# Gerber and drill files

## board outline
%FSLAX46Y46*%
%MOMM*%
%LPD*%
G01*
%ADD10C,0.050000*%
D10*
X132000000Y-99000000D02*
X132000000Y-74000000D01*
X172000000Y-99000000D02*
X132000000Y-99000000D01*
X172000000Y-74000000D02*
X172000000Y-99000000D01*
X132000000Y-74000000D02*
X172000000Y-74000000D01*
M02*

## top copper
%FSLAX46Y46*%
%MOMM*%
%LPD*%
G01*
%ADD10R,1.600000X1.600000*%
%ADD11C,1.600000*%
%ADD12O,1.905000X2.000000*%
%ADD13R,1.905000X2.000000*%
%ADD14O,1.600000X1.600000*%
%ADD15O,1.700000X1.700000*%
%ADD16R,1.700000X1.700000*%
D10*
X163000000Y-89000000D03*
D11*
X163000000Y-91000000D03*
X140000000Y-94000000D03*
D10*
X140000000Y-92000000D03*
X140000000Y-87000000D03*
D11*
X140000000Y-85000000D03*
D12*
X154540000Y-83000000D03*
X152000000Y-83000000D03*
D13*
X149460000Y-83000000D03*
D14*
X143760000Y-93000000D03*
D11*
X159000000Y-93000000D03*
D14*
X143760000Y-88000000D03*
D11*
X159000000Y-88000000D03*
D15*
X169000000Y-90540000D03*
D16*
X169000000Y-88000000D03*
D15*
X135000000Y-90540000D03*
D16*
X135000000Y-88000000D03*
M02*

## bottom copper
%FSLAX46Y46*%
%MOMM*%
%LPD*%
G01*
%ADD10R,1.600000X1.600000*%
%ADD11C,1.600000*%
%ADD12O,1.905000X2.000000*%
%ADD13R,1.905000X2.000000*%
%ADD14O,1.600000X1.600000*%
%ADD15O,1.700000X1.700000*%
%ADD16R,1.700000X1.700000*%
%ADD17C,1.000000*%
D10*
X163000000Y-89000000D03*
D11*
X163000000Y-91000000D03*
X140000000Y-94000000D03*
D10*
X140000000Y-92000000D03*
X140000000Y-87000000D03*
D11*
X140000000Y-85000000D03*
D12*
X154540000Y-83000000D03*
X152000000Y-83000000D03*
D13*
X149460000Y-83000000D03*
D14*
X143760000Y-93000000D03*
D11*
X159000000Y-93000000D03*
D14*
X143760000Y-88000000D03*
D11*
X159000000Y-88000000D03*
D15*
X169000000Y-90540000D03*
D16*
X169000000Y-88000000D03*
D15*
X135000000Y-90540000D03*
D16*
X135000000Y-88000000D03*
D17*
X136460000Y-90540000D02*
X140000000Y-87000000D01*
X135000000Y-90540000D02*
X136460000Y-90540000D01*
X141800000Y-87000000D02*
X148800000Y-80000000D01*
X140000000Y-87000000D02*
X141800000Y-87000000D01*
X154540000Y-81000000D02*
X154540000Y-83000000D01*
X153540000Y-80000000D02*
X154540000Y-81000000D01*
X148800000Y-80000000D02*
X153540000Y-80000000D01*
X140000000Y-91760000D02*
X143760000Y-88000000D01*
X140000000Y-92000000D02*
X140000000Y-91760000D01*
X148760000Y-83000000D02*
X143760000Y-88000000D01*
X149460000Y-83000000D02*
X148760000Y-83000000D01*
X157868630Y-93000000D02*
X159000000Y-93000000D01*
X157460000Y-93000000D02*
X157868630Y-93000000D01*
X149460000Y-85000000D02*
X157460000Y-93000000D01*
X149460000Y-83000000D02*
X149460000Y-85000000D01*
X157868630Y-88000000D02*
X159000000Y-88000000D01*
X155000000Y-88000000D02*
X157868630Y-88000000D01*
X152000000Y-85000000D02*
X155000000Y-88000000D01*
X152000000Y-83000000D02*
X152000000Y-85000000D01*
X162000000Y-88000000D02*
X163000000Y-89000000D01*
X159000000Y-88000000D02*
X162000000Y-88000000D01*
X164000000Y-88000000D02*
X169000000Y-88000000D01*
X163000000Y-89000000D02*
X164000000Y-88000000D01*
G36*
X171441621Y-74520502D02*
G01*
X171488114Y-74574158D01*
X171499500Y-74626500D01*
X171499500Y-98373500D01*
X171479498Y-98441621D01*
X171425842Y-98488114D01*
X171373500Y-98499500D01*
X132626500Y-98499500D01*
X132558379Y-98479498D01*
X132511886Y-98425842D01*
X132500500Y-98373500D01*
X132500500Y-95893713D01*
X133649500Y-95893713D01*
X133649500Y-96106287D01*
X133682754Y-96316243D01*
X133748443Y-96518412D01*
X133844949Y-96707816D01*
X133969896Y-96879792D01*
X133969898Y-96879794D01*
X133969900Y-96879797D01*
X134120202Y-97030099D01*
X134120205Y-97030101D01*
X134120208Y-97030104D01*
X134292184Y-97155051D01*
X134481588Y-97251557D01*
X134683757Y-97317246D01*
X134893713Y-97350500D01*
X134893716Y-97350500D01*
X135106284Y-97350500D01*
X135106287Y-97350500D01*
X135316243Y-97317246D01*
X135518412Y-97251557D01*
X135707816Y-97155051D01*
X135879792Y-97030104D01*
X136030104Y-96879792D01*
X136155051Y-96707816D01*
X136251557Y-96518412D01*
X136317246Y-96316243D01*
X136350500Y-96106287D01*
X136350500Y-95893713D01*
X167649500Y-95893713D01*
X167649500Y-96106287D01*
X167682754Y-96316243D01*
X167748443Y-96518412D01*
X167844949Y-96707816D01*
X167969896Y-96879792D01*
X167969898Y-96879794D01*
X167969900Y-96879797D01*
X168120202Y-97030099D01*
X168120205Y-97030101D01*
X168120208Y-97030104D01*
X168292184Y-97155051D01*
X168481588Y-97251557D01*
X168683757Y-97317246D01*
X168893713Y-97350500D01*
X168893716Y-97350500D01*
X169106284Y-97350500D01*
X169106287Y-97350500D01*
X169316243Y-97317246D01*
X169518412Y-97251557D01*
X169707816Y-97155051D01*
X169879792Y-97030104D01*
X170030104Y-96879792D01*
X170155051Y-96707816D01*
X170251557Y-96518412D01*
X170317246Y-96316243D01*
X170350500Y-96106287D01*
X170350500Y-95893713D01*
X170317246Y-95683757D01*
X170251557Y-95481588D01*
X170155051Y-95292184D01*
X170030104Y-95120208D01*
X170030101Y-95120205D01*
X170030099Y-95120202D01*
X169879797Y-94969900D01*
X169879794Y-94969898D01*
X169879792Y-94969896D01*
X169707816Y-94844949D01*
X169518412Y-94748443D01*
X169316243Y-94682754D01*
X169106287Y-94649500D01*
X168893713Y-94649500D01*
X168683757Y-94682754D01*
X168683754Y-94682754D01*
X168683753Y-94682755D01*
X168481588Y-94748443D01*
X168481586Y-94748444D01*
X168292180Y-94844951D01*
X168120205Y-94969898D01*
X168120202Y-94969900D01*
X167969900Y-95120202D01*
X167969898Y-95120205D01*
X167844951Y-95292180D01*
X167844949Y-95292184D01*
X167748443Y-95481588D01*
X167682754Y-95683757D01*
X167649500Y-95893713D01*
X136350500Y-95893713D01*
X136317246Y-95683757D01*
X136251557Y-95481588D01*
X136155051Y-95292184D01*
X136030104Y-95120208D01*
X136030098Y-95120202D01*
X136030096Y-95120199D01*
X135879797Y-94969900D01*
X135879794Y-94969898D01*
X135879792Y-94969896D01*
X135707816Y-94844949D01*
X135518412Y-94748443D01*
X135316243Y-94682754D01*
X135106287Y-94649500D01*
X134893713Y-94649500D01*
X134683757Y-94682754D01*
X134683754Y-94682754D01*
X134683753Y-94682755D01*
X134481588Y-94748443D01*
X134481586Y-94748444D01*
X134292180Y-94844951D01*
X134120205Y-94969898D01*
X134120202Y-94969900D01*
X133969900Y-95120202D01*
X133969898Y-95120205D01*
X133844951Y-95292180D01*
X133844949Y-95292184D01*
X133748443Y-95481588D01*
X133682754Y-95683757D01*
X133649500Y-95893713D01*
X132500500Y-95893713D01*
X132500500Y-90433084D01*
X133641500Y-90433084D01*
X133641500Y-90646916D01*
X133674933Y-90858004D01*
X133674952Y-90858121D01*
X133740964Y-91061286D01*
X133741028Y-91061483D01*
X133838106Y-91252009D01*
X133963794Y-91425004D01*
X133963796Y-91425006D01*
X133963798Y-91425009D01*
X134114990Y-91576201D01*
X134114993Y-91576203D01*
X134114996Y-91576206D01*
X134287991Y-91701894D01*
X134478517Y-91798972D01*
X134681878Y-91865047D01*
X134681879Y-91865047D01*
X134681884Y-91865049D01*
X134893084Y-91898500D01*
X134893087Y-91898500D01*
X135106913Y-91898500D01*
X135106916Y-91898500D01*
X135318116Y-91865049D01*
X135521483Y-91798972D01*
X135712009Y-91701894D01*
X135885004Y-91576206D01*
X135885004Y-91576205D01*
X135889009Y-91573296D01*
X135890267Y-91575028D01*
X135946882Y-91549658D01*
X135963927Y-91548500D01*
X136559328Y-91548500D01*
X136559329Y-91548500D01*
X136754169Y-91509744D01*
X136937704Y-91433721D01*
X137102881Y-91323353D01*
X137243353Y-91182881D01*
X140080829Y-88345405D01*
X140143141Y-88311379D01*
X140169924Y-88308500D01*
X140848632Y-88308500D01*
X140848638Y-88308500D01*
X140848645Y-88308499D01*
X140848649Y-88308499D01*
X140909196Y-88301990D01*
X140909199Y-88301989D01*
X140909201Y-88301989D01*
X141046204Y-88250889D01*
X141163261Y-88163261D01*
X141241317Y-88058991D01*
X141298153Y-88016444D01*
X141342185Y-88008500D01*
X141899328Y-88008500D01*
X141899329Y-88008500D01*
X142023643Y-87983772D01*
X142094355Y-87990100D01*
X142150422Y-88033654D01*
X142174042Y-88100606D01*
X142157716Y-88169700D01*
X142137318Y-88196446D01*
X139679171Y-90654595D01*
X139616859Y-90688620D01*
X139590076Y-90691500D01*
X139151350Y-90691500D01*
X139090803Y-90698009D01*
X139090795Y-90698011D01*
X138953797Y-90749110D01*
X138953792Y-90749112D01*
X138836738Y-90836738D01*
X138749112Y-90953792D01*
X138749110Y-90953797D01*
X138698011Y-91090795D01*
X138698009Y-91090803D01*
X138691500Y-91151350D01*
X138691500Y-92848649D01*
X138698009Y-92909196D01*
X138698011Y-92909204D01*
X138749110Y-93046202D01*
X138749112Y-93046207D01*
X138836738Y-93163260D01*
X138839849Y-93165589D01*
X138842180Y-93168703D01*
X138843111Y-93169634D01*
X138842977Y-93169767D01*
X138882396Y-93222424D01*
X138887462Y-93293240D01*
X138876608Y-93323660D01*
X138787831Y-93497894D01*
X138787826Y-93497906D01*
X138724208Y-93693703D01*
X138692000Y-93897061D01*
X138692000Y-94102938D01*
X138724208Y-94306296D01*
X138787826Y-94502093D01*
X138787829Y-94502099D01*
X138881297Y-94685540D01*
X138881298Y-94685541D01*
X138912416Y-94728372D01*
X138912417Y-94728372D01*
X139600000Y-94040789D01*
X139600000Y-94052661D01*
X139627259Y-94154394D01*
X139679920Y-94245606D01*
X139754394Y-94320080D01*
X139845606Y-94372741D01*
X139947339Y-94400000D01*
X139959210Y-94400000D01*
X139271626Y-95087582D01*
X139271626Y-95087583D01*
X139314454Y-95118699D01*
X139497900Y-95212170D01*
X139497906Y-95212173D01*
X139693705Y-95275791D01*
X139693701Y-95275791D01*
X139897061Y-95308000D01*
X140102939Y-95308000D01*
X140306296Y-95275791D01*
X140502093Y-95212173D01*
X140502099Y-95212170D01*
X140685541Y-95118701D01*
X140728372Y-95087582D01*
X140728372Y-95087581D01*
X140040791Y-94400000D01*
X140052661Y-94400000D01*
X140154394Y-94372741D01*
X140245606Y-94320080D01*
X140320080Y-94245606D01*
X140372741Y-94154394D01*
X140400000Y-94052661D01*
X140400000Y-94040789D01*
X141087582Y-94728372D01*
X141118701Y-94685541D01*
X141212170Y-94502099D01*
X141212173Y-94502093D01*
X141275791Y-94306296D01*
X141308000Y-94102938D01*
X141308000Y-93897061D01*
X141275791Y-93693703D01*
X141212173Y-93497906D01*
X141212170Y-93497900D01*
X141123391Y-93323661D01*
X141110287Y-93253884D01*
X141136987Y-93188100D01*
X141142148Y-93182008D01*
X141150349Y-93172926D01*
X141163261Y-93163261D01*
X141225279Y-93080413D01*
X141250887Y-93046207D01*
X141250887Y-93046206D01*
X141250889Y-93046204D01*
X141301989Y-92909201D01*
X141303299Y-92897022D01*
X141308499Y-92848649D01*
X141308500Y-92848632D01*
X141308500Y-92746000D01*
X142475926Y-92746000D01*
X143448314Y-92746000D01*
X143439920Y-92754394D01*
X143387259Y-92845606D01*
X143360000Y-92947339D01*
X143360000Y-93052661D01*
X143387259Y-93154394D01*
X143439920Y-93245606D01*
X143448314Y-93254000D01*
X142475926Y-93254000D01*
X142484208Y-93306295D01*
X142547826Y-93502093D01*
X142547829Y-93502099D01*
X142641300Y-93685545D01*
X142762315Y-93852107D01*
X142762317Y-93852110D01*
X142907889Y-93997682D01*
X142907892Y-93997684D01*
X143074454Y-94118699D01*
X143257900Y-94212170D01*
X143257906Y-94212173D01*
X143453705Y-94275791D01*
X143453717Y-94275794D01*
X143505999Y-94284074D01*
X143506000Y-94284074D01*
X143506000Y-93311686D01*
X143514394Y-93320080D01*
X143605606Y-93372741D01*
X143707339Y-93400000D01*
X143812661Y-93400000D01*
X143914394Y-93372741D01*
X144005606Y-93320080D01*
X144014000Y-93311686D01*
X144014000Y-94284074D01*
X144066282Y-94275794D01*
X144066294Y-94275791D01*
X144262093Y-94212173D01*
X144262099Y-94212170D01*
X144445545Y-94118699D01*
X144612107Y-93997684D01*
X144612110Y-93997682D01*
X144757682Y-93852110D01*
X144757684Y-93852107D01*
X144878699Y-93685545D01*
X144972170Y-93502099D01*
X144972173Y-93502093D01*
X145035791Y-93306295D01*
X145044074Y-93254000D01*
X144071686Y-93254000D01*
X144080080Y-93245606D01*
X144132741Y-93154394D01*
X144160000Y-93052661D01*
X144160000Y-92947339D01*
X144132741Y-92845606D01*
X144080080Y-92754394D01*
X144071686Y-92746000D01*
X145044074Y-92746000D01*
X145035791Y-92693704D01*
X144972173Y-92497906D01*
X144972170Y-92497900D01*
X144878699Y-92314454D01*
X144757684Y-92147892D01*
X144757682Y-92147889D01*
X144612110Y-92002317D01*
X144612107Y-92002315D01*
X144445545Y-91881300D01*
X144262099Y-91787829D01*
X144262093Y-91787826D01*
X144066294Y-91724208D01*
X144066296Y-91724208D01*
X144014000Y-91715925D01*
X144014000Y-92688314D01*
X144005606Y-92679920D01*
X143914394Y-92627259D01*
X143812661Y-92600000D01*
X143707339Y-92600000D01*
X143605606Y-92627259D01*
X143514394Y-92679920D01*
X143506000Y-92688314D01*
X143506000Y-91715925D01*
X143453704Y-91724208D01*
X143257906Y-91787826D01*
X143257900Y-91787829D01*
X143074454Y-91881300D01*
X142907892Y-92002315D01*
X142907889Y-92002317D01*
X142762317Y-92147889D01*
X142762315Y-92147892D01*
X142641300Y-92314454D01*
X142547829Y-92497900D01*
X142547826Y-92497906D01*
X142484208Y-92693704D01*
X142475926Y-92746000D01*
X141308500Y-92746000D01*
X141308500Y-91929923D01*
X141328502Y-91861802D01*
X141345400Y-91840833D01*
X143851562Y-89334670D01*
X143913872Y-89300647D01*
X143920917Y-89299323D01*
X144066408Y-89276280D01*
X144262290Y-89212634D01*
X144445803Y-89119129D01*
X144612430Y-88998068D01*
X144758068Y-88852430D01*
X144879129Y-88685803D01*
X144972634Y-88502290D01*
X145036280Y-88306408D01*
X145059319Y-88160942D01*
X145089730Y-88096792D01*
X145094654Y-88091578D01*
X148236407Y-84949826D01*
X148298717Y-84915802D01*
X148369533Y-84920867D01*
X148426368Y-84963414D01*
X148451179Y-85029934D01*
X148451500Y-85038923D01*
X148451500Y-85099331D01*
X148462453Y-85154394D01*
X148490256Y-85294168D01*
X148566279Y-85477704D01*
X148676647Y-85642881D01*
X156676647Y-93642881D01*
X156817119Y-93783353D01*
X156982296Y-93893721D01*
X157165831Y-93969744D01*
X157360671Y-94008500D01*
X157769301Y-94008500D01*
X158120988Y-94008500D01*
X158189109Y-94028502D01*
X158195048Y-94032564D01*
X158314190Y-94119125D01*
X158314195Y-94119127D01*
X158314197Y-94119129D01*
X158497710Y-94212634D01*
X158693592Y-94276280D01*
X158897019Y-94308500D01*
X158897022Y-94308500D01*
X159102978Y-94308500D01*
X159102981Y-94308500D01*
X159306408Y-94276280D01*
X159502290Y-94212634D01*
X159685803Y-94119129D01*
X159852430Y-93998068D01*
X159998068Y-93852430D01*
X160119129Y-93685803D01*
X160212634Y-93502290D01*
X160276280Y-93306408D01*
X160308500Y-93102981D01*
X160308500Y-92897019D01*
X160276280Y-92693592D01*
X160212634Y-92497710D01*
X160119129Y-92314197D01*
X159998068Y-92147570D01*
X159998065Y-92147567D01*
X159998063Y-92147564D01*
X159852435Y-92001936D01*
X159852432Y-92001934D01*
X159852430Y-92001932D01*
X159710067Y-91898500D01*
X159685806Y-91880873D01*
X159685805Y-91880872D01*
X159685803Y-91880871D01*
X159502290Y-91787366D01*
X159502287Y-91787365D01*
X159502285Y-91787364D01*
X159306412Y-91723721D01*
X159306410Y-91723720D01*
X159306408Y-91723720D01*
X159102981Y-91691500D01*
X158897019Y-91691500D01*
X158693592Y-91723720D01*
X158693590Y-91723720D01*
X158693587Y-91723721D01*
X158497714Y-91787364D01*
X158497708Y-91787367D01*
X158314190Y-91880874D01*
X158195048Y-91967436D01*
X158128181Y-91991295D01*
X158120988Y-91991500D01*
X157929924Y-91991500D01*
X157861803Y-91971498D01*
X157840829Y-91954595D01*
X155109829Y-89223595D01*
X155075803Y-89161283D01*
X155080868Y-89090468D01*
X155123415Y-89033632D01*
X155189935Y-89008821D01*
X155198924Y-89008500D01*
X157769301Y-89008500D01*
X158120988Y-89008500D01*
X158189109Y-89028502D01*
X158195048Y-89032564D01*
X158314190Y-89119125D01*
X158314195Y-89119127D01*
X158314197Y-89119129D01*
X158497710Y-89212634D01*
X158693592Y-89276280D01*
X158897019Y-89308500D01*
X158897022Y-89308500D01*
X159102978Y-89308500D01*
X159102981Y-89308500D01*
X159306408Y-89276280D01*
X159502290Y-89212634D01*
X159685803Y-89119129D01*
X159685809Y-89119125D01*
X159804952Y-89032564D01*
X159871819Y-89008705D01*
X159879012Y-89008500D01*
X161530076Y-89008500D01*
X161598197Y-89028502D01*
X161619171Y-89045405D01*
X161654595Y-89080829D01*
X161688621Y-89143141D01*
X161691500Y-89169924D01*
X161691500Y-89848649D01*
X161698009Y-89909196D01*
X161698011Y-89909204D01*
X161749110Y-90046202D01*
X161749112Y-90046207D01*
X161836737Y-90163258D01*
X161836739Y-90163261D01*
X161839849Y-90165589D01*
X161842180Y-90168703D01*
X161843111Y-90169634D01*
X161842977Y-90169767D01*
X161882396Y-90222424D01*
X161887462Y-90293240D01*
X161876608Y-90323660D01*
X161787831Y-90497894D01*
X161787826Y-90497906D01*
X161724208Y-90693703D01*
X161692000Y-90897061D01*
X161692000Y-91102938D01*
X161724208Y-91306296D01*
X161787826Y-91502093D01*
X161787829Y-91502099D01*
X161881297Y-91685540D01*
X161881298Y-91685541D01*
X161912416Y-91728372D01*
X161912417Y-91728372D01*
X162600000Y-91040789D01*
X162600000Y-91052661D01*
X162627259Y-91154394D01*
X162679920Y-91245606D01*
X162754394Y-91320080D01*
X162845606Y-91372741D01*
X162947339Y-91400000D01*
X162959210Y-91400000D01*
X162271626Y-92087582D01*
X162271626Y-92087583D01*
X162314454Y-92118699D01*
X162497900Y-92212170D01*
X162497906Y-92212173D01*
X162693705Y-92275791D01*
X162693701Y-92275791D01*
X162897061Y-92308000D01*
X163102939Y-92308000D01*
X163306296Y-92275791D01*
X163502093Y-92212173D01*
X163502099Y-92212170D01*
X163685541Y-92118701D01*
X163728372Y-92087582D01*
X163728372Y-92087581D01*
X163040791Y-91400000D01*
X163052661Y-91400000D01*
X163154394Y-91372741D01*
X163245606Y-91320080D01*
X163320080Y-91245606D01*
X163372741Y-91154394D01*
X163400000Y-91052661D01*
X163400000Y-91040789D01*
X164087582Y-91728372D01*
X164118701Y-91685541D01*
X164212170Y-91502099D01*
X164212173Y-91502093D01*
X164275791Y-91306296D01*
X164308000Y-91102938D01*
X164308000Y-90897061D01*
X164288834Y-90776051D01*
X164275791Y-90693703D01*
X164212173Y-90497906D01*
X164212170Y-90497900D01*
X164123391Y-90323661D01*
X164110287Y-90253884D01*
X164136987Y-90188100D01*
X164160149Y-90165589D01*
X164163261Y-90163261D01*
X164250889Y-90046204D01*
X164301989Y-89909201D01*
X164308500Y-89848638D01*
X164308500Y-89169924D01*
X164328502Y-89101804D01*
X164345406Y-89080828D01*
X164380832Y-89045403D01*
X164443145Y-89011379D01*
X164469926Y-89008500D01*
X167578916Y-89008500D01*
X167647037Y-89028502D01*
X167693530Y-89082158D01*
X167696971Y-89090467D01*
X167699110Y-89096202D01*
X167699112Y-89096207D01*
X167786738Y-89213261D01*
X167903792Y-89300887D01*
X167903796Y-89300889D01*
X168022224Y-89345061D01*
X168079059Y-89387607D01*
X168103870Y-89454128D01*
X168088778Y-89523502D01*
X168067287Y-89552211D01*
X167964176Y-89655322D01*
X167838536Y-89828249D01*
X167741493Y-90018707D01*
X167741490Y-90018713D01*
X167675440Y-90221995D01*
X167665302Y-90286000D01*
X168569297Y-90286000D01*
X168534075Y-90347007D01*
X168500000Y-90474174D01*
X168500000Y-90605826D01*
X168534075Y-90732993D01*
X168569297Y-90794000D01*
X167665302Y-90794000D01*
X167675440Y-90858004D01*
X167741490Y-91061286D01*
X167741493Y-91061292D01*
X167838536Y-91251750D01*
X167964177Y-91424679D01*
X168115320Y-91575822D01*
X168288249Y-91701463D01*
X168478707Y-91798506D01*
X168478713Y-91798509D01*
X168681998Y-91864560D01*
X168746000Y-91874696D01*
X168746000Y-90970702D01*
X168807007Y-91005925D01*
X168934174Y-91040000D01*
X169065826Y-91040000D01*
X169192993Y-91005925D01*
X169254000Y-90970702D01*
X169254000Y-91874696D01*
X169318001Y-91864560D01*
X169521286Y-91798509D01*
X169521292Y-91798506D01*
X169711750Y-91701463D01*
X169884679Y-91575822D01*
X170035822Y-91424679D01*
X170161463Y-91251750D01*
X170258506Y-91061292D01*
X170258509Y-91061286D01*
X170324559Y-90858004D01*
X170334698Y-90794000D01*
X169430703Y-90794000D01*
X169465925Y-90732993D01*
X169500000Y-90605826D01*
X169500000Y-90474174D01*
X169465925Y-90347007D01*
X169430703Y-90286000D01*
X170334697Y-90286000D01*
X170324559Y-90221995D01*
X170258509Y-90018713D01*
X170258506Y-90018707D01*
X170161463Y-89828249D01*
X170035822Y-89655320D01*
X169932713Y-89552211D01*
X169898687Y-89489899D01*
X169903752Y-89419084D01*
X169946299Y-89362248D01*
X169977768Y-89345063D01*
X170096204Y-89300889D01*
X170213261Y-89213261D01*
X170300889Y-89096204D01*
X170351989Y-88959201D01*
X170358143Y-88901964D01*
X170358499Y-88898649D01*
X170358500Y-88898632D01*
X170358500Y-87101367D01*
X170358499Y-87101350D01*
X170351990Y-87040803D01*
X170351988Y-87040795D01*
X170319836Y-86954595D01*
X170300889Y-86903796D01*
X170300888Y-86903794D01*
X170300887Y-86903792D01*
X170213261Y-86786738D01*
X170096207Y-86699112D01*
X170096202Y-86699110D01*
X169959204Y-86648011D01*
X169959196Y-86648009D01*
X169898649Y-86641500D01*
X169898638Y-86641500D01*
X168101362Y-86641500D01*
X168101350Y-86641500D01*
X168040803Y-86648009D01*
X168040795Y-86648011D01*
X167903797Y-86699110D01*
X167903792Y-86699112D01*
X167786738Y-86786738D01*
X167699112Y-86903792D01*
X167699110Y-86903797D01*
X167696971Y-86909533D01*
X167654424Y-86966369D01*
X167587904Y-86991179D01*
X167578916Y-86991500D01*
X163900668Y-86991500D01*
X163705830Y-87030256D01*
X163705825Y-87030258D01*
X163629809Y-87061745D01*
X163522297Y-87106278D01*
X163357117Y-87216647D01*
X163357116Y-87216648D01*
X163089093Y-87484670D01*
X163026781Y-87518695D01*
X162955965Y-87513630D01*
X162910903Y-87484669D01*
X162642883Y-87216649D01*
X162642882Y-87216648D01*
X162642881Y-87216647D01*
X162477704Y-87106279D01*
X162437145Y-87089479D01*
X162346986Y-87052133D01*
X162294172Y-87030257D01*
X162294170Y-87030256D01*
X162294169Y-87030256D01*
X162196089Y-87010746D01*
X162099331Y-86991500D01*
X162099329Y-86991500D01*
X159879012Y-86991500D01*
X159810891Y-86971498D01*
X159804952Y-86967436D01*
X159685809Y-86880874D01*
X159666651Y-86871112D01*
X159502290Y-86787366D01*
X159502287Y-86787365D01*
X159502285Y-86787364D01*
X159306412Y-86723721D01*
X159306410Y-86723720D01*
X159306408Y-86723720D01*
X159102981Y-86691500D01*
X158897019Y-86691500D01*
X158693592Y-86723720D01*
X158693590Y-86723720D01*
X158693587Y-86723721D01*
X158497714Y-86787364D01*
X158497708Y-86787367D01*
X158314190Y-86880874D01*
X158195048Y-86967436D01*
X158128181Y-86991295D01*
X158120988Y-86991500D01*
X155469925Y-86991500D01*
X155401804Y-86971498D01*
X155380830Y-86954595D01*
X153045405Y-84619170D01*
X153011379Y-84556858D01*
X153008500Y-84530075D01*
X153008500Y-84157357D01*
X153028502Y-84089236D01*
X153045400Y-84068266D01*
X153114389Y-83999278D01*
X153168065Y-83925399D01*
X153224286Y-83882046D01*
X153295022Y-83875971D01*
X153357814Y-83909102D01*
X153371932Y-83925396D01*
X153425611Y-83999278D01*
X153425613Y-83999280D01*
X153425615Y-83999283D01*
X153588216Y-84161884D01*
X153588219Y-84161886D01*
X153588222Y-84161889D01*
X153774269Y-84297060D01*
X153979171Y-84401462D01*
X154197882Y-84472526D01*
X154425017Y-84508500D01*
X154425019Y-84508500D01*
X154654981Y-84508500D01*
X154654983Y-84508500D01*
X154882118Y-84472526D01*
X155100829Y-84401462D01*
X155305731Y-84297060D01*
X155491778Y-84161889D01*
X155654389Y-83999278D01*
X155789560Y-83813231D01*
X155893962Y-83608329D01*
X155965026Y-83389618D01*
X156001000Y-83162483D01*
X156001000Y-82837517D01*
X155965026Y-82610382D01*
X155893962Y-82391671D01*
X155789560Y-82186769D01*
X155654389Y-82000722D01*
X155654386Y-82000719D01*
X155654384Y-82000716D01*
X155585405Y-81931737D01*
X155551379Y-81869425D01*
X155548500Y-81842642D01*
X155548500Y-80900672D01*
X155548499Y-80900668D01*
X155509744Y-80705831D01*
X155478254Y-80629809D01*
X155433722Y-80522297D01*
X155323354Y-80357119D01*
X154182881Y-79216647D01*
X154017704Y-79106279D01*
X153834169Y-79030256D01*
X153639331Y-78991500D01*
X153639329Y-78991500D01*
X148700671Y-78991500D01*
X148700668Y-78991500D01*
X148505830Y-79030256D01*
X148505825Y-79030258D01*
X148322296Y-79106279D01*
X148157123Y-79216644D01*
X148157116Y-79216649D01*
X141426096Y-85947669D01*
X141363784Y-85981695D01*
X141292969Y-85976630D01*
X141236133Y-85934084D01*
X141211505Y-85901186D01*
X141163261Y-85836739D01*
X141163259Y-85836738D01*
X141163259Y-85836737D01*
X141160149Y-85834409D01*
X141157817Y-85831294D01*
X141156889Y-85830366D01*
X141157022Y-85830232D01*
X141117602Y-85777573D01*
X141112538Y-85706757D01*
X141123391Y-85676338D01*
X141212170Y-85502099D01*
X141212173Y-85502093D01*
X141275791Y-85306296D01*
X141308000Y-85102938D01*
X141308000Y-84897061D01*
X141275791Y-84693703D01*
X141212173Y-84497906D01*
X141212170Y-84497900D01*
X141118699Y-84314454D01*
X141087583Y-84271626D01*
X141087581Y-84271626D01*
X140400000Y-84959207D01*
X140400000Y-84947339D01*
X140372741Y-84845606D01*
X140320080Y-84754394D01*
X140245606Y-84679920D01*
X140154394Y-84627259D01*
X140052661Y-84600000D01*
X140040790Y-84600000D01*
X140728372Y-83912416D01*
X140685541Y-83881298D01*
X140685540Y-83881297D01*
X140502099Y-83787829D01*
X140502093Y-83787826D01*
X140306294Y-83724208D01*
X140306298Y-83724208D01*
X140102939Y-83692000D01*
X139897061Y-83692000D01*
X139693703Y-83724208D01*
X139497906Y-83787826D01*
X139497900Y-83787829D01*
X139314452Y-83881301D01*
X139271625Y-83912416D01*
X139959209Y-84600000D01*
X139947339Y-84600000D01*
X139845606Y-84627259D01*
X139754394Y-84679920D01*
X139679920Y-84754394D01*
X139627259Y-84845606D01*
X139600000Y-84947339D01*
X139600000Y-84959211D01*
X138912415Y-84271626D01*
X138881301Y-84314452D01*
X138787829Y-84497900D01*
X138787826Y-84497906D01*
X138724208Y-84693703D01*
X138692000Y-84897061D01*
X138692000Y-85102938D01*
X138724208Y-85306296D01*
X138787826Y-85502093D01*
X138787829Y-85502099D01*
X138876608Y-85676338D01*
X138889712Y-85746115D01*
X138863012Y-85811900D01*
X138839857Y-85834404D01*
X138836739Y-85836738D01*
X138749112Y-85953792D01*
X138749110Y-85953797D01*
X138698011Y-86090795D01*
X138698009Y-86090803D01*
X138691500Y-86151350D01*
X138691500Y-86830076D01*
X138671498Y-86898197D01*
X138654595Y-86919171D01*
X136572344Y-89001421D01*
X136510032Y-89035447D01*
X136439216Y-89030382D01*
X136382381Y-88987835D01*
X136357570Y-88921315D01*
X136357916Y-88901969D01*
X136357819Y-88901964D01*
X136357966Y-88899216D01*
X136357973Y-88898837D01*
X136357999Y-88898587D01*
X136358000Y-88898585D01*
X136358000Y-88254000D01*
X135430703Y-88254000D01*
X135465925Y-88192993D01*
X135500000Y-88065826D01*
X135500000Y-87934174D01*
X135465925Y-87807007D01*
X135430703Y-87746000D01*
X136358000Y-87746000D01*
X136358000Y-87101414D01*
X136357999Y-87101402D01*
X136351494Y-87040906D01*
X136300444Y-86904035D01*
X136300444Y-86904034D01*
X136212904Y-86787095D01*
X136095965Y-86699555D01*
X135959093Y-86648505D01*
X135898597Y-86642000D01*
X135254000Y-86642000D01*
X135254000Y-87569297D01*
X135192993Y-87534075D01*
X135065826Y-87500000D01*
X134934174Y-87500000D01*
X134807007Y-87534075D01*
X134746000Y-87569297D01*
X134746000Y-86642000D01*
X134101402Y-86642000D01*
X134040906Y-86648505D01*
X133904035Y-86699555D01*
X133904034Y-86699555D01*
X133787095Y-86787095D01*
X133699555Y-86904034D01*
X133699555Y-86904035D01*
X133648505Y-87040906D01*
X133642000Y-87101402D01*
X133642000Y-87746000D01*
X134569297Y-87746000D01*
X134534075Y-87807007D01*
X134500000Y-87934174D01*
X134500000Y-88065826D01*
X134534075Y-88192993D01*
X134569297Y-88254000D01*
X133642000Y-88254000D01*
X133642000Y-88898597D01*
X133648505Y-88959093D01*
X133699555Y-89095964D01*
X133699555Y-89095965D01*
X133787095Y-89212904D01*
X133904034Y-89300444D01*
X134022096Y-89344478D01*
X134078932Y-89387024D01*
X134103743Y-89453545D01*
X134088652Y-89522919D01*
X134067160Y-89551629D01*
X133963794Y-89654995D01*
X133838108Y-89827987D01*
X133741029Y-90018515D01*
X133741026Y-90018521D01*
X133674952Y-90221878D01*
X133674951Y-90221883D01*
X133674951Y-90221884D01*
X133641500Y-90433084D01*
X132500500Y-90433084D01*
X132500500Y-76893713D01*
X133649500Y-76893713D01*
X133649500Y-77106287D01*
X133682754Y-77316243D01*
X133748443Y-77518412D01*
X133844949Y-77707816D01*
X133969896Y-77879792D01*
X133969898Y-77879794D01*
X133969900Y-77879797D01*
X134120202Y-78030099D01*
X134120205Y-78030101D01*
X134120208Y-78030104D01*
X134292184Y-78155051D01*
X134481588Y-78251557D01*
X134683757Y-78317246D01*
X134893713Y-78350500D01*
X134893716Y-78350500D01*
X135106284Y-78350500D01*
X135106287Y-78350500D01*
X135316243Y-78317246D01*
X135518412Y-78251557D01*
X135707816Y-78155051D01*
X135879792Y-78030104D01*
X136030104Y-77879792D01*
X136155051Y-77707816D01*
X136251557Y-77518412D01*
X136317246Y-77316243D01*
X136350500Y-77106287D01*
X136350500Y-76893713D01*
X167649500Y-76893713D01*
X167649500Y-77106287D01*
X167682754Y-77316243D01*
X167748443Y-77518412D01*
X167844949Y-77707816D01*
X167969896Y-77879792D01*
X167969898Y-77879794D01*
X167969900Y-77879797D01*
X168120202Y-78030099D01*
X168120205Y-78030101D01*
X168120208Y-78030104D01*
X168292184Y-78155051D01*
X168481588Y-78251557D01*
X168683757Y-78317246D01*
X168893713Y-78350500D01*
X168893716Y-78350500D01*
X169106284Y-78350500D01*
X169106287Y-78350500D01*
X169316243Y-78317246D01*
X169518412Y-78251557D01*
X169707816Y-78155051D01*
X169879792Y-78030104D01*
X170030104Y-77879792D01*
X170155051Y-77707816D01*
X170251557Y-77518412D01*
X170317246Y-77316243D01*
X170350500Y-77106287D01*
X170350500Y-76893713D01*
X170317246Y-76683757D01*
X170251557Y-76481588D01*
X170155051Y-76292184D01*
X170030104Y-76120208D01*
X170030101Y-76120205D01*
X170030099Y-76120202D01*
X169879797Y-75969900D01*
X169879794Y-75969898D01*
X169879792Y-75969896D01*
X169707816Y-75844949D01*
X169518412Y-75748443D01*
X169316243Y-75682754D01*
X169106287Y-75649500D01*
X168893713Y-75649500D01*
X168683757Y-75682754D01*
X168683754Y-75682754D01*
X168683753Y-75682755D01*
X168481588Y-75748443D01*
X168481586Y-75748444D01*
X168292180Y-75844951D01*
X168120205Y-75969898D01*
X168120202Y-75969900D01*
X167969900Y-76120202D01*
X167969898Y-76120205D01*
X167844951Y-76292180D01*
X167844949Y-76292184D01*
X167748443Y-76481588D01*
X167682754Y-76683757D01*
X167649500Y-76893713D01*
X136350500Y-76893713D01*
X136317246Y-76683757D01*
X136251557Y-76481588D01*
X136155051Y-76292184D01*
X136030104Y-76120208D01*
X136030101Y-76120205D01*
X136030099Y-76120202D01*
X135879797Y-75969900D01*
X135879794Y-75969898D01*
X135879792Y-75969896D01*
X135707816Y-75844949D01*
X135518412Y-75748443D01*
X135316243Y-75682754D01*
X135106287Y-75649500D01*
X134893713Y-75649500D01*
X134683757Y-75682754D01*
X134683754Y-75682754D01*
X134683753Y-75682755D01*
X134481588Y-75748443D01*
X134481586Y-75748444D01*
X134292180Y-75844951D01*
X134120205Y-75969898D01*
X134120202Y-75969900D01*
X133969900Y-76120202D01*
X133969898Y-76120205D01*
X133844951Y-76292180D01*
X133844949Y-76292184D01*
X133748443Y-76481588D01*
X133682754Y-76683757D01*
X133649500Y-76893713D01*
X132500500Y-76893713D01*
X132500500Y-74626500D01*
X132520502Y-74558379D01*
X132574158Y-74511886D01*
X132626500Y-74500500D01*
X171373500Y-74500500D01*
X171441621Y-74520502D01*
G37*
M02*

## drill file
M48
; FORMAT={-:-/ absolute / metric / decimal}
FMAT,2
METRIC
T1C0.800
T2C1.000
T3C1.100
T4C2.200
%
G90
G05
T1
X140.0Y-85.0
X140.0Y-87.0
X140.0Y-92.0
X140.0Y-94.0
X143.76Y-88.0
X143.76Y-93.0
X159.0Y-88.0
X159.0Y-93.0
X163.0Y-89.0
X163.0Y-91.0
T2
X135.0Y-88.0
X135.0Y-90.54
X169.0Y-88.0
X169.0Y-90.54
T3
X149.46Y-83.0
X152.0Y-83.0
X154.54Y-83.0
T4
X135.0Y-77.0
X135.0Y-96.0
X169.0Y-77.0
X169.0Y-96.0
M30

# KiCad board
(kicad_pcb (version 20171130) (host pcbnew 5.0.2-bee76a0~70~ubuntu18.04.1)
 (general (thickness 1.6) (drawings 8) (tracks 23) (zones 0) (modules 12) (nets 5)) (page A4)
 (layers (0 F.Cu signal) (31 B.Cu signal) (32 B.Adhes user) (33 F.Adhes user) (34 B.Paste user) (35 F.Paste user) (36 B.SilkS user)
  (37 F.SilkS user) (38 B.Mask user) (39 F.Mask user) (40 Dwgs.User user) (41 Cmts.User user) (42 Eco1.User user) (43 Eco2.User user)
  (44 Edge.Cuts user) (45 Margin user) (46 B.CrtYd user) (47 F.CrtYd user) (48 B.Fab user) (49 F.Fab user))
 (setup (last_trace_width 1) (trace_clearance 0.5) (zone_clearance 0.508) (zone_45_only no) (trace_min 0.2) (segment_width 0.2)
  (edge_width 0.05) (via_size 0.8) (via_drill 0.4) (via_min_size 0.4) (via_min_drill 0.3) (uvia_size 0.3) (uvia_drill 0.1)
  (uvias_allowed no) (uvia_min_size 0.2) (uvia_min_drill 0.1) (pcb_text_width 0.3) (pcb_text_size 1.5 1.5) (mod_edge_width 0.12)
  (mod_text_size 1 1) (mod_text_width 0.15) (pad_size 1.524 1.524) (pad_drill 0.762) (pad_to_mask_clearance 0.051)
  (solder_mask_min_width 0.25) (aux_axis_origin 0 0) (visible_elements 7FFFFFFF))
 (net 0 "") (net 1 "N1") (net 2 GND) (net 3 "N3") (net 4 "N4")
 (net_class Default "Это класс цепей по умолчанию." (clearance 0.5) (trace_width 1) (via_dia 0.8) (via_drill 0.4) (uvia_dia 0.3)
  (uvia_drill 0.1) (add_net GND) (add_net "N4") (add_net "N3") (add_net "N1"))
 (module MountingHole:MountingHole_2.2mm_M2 (layer F.Cu) (at 169 77)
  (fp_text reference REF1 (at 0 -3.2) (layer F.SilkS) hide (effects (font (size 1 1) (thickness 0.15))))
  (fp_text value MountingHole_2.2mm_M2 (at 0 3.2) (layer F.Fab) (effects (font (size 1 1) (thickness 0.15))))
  (pad 1 np_thru_hole circle (at 0 0) (size 2.2 2.2) (drill 2.2) (layers *.Cu *.Mask)))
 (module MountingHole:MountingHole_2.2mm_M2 (layer F.Cu) (at 169 96)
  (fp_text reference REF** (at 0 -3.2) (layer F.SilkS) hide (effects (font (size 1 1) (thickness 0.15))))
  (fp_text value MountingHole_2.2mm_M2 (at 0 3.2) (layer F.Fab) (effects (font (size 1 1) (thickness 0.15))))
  (pad 1 np_thru_hole circle (at 0 0) (size 2.2 2.2) (drill 2.2) (layers *.Cu *.Mask)))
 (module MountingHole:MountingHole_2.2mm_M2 (layer F.Cu) (at 135 77)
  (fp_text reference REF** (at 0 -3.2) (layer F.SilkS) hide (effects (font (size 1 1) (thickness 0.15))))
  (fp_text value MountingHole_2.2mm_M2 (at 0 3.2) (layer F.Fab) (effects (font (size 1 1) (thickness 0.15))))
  (pad 1 np_thru_hole circle (at 0 0) (size 2.2 2.2) (drill 2.2) (layers *.Cu *.Mask)))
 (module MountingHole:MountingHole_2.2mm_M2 (layer F.Cu) (at 135 96)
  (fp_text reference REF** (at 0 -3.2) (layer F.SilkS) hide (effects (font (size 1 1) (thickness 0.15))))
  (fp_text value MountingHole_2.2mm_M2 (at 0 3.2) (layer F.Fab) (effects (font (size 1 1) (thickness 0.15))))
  (pad 1 np_thru_hole circle (at 0 0) (size 2.2 2.2) (drill 2.2) (layers *.Cu *.Mask)))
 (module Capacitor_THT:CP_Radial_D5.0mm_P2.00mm (layer F.Cu) (at 163 89 270)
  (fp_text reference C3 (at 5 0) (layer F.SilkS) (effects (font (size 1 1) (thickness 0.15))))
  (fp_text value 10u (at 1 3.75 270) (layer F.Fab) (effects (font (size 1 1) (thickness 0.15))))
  (pad 1 thru_hole rect (at 0 0 270) (size 1.6 1.6) (drill 0.8) (layers *.Cu *.Mask) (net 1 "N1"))
  (pad 2 thru_hole circle (at 2 0 270) (size 1.6 1.6) (drill 0.8) (layers *.Cu *.Mask) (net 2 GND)))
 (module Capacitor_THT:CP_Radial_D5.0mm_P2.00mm (layer F.Cu) (at 140 92 270)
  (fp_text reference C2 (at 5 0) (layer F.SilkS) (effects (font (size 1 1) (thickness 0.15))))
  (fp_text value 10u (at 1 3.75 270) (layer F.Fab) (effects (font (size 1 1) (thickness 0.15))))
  (pad 2 thru_hole circle (at 2 0 270) (size 1.6 1.6) (drill 0.8) (layers *.Cu *.Mask) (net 2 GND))
  (pad 1 thru_hole rect (at 0 0 270) (size 1.6 1.6) (drill 0.8) (layers *.Cu *.Mask) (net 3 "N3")))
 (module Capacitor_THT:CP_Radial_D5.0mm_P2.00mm (layer F.Cu) (at 140 87 90)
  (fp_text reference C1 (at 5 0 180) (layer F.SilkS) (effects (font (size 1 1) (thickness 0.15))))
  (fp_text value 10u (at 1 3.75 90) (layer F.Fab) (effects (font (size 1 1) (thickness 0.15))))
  (pad 1 thru_hole rect (at 0 0 90) (size 1.6 1.6) (drill 0.8) (layers *.Cu *.Mask) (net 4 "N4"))
  (pad 2 thru_hole circle (at 2 0 90) (size 1.6 1.6) (drill 0.8) (layers *.Cu *.Mask) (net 2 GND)))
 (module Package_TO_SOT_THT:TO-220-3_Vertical (layer F.Cu) (at 149.46 83)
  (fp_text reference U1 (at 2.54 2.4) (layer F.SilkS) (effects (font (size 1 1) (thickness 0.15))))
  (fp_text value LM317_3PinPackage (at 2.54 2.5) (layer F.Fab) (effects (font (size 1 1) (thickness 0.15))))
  (pad 3 thru_hole oval (at 5.08 0) (size 1.905 2) (drill 1.1) (layers *.Cu *.Mask) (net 4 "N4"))
  (pad 2 thru_hole oval (at 2.54 0) (size 1.905 2) (drill 1.1) (layers *.Cu *.Mask) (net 1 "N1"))
  (pad 1 thru_hole rect (at 0 0) (size 1.905 2) (drill 1.1) (layers *.Cu *.Mask) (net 3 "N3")))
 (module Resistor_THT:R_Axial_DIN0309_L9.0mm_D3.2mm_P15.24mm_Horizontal (layer F.Cu) (at 159 93 180)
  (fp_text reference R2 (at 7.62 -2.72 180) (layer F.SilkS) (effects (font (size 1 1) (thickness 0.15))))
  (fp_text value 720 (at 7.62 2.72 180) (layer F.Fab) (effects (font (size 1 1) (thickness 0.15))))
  (pad 2 thru_hole oval (at 15.24 0 180) (size 1.6 1.6) (drill 0.8) (layers *.Cu *.Mask) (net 2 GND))
  (pad 1 thru_hole circle (at 0 0 180) (size 1.6 1.6) (drill 0.8) (layers *.Cu *.Mask) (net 3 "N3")))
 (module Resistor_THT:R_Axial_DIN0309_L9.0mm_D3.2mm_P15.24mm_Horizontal (layer F.Cu) (at 159 88 180)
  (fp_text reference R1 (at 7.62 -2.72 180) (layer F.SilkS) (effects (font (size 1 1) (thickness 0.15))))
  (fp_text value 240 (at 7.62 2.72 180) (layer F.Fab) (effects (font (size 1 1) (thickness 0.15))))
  (pad 2 thru_hole oval (at 15.24 0 180) (size 1.6 1.6) (drill 0.8) (layers *.Cu *.Mask) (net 3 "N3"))
  (pad 1 thru_hole circle (at 0 0 180) (size 1.6 1.6) (drill 0.8) (layers *.Cu *.Mask) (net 1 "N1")))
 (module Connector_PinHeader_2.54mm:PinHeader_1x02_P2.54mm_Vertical (layer F.Cu) (at 169 88)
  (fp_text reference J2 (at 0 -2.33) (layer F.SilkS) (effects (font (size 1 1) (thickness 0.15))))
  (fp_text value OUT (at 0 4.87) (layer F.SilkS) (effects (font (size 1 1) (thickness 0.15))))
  (pad 2 thru_hole oval (at 0 2.54) (size 1.7 1.7) (drill 1) (layers *.Cu *.Mask) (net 2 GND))
  (pad 1 thru_hole rect (at 0 0) (size 1.7 1.7) (drill 1) (layers *.Cu *.Mask) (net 1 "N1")))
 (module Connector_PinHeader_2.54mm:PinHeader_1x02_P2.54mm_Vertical (layer F.Cu) (at 135 88)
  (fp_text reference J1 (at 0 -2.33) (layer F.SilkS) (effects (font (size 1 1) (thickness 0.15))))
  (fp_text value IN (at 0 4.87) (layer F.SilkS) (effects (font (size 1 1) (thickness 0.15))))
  (pad 2 thru_hole oval (at 0 2.54) (size 1.7 1.7) (drill 1) (layers *.Cu *.Mask) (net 4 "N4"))
  (pad 1 thru_hole rect (at 0 0) (size 1.7 1.7) (drill 1) (layers *.Cu *.Mask) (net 2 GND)))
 (gr_line (start 132 99) (end 132 74) (layer Edge.Cuts) (width 0.05))
 (gr_line (start 172 99) (end 132 99) (layer Edge.Cuts) (width 0.05))
 (gr_line (start 172 74) (end 172 99) (layer Edge.Cuts) (width 0.05))
 (gr_line (start 132 74) (end 172 74) (layer Edge.Cuts) (width 0.05))
 (segment (start 136.46 90.54) (end 140 87) (width 1) (layer B.Cu) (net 4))
 (segment (start 135 90.54) (end 136.46 90.54) (width 1) (layer B.Cu) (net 4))
 (segment (start 141.8 87) (end 148.8 80) (width 1) (layer B.Cu) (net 4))
 (segment (start 140 87) (end 141.8 87) (width 1) (layer B.Cu) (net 4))
 (segment (start 154.54 81) (end 154.54 83) (width 1) (layer B.Cu) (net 4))
 (segment (start 153.54 80) (end 154.54 81) (width 1) (layer B.Cu) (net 4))
 (segment (start 148.8 80) (end 153.54 80) (width 1) (layer B.Cu) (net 4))
 (segment (start 140 91.76) (end 143.76 88) (width 1) (layer B.Cu) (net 3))
 (segment (start 140 92) (end 140 91.76) (width 1) (layer B.Cu) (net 3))
 (segment (start 148.76 83) (end 143.76 88) (width 1) (layer B.Cu) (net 3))
 (segment (start 149.46 83) (end 148.76 83) (width 1) (layer B.Cu) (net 3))
 (segment (start 157.86863 93) (end 159 93) (width 1) (layer B.Cu) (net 3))
 (segment (start 157.46 93) (end 157.86863 93) (width 1) (layer B.Cu) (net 3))
 (segment (start 149.46 85) (end 157.46 93) (width 1) (layer B.Cu) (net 3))
 (segment (start 149.46 83) (end 149.46 85) (width 1) (layer B.Cu) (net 3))
 (segment (start 157.86863 88) (end 159 88) (width 1) (layer B.Cu) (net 1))
 (segment (start 155 88) (end 157.86863 88) (width 1) (layer B.Cu) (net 1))
 (segment (start 152 85) (end 155 88) (width 1) (layer B.Cu) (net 1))
 (segment (start 152 83) (end 152 85) (width 1) (layer B.Cu) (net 1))
 (segment (start 162 88) (end 163 89) (width 1) (layer B.Cu) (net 1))
 (segment (start 159 88) (end 162 88) (width 1) (layer B.Cu) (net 1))
 (segment (start 164 88) (end 169 88) (width 1) (layer B.Cu) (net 1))
 (segment (start 163 89) (end 164 88) (width 1) (layer B.Cu) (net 1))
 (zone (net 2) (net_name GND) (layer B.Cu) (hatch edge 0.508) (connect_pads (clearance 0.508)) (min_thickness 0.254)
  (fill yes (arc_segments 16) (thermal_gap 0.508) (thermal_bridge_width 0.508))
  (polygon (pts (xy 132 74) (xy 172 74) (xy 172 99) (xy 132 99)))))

